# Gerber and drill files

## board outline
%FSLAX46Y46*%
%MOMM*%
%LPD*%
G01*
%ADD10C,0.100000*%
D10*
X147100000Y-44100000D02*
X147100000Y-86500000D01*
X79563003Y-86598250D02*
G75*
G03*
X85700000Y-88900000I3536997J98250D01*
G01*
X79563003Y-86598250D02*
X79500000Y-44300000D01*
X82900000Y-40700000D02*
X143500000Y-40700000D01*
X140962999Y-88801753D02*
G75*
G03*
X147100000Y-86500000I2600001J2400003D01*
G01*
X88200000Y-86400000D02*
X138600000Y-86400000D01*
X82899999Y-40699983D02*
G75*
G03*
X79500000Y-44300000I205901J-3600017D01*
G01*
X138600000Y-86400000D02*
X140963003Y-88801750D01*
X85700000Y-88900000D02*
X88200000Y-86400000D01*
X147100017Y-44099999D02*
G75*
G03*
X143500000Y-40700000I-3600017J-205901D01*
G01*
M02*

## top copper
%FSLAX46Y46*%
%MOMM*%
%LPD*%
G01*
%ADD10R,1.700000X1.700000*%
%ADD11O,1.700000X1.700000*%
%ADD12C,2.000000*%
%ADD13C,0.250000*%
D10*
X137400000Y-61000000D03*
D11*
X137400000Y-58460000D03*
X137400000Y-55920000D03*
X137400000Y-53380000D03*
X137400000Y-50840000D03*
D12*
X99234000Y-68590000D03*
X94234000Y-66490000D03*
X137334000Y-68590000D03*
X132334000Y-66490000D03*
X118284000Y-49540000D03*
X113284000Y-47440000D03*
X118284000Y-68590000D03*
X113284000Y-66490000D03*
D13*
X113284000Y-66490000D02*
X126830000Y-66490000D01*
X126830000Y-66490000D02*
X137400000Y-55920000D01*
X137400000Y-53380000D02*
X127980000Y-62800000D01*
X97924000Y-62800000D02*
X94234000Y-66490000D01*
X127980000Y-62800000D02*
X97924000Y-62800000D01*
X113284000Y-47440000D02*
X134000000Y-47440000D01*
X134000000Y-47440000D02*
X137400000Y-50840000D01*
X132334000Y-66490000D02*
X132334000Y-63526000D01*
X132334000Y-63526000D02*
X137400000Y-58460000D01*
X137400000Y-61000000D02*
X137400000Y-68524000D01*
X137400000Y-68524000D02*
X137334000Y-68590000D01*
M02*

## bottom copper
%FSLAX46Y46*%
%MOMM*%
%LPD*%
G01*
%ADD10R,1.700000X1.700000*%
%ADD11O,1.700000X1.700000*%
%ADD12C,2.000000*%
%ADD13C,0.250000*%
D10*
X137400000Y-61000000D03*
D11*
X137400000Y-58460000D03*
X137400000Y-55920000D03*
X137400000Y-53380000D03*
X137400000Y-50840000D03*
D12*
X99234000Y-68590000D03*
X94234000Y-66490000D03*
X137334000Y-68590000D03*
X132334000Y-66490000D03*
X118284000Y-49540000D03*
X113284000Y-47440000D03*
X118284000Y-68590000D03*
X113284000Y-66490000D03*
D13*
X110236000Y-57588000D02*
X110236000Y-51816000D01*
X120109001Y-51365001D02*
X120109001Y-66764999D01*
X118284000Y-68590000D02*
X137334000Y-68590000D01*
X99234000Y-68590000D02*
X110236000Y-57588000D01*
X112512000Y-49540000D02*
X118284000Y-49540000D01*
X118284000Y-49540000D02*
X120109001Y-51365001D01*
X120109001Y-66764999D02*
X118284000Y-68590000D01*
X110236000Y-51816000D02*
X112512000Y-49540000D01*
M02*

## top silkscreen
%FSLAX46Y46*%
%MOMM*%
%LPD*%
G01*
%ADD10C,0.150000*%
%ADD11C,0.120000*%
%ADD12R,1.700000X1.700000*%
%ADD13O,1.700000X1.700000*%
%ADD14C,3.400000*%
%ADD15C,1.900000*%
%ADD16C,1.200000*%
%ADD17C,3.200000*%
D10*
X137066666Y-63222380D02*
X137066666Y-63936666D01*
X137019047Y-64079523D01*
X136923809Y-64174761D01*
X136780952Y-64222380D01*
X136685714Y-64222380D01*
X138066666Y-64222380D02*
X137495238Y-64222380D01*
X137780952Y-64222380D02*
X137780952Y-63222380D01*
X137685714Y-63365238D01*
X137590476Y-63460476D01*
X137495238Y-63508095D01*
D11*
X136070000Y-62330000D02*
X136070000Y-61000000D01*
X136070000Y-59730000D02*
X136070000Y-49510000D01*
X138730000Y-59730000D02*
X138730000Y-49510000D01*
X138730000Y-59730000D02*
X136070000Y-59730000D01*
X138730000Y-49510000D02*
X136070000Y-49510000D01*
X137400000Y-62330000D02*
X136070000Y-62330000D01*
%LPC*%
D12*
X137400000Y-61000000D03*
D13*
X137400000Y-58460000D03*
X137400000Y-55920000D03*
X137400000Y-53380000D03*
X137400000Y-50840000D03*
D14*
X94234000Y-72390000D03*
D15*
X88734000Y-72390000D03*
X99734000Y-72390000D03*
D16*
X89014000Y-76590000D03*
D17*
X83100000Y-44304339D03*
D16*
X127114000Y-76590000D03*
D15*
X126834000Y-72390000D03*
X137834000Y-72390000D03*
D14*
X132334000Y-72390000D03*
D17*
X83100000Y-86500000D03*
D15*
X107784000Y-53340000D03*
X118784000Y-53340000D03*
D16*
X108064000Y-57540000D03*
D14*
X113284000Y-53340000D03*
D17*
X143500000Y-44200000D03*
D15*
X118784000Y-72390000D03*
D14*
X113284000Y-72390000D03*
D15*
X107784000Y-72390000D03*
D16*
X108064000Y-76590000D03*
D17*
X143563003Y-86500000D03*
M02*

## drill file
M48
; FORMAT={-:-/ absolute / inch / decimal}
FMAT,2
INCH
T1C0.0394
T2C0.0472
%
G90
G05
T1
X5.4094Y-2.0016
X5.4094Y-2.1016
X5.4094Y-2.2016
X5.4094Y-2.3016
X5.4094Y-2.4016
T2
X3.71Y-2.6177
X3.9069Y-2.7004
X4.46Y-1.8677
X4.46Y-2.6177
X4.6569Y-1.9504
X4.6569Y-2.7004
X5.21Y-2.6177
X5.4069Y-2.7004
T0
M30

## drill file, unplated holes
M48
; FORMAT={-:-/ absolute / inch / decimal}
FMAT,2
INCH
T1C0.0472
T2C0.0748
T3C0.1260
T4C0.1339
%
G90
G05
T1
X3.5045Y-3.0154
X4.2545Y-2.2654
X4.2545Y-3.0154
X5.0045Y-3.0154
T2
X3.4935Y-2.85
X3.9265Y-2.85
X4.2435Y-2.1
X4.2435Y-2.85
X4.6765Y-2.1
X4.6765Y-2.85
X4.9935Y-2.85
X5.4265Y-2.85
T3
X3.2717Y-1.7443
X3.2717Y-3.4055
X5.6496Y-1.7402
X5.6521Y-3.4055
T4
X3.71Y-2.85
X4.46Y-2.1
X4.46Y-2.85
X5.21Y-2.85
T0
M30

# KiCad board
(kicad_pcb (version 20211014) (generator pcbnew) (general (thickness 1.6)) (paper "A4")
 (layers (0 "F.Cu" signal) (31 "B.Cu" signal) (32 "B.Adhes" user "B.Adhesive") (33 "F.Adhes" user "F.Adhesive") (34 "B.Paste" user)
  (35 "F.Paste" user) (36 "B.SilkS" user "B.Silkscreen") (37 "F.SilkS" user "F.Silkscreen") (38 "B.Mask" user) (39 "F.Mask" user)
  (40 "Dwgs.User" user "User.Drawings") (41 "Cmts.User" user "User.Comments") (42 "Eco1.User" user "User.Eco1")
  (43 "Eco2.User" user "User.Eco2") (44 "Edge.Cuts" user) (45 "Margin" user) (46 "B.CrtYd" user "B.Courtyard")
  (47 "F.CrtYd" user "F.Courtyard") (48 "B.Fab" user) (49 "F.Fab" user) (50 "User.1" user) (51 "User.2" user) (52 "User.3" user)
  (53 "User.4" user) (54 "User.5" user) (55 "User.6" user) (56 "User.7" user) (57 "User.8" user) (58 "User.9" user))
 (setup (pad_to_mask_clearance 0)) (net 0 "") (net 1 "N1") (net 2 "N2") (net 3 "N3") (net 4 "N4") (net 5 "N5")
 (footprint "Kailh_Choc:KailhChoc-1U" (layer "F.Cu") (at 94.234 72.39)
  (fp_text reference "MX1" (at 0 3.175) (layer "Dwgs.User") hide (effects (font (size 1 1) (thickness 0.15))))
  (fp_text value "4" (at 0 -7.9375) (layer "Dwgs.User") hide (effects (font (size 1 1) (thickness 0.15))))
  (pad "" np_thru_hole circle (at 0 0) (size 3.4 3.4) (drill 3.4) (layers *.Cu *.Mask))
  (pad "" np_thru_hole circle (at -5.5 0 48.1) (size 1.9 1.9) (drill 1.9) (layers *.Cu *.Mask))
  (pad "" np_thru_hole circle (at 5.5 0 48.1) (size 1.9 1.9) (drill 1.9) (layers *.Cu *.Mask))
  (pad "" np_thru_hole circle (at -5.22 4.2) (size 1.2 1.2) (drill 1.2) (layers *.Cu *.Mask))
  (pad "1" thru_hole circle (at 5 -3.8) (size 2 2) (drill 1.2) (layers *.Cu "B.Mask") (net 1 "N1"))
  (pad "2" thru_hole circle (at 0 -5.9) (size 2 2) (drill 1.2) (layers *.Cu "B.Mask") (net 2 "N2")))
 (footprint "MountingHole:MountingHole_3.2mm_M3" (layer "F.Cu") (at 83.1 44.304339)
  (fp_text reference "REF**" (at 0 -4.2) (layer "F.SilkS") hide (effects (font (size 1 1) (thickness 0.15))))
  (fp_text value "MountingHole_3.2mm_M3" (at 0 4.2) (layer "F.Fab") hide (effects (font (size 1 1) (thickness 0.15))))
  (pad "" np_thru_hole circle locked (at 0 0) (size 3.2 3.2) (drill 3.2) (layers F&B.Cu *.Mask)))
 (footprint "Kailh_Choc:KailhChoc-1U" (layer "F.Cu") (at 132.334 72.39)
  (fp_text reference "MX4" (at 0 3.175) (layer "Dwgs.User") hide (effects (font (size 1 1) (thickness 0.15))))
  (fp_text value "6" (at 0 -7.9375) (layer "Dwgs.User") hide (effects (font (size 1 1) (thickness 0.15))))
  (pad "" np_thru_hole circle (at -5.22 4.2) (size 1.2 1.2) (drill 1.2) (layers *.Cu *.Mask))
  (pad "" np_thru_hole circle (at -5.5 0 48.1) (size 1.9 1.9) (drill 1.9) (layers *.Cu *.Mask))
  (pad "" np_thru_hole circle (at 5.5 0 48.1) (size 1.9 1.9) (drill 1.9) (layers *.Cu *.Mask))
  (pad "" np_thru_hole circle (at 0 0) (size 3.4 3.4) (drill 3.4) (layers *.Cu *.Mask))
  (pad "1" thru_hole circle (at 5 -3.8) (size 2 2) (drill 1.2) (layers *.Cu "B.Mask") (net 1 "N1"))
  (pad "2" thru_hole circle (at 0 -5.9) (size 2 2) (drill 1.2) (layers *.Cu "B.Mask") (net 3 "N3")))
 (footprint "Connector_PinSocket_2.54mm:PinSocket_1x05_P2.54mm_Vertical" (layer "F.Cu") (at 137.4 61 180)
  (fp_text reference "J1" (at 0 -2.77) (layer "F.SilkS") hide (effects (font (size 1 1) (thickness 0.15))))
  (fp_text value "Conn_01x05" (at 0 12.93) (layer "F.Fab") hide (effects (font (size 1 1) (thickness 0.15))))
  (fp_line (start -1.33 1.27) (end 1.33 1.27) (layer "F.SilkS") (width 0.12))
  (fp_line (start -1.33 11.49) (end 1.33 11.49) (layer "F.SilkS") (width 0.12))
  (fp_line (start 1.33 1.27) (end 1.33 11.49) (layer "F.SilkS") (width 0.12))
  (fp_line (start 0 -1.33) (end 1.33 -1.33) (layer "F.SilkS") (width 0.12))
  (fp_line (start -1.33 1.27) (end -1.33 11.49) (layer "F.SilkS") (width 0.12))
  (fp_line (start 1.33 -1.33) (end 1.33 0) (layer "F.SilkS") (width 0.12))
  (pad "1" thru_hole rect (at 0 0 180) (size 1.7 1.7) (drill 1) (layers *.Cu *.Mask) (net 1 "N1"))
  (pad "2" thru_hole oval (at 0 2.54 180) (size 1.7 1.7) (drill 1) (layers *.Cu *.Mask) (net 3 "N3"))
  (pad "3" thru_hole oval (at 0 5.08 180) (size 1.7 1.7) (drill 1) (layers *.Cu *.Mask) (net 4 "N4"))
  (pad "4" thru_hole oval (at 0 7.62 180) (size 1.7 1.7) (drill 1) (layers *.Cu *.Mask) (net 2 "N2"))
  (pad "5" thru_hole oval (at 0 10.16 180) (size 1.7 1.7) (drill 1) (layers *.Cu *.Mask) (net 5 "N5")))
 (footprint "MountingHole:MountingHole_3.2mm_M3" (layer "F.Cu") (at 83.1 86.5)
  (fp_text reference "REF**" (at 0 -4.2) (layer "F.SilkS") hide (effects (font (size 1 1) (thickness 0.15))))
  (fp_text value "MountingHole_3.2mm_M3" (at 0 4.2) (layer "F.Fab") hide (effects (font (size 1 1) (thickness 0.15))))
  (pad "" np_thru_hole circle locked (at 0 0) (size 3.2 3.2) (drill 3.2) (layers *.Cu *.Mask)))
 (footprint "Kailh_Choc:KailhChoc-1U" (layer "F.Cu") (at 113.284 53.34)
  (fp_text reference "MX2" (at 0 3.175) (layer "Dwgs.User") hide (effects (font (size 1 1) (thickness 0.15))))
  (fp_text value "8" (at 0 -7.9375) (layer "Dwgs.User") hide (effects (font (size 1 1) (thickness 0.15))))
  (pad "" np_thru_hole circle (at -5.5 0 48.1) (size 1.9 1.9) (drill 1.9) (layers *.Cu *.Mask))
  (pad "" np_thru_hole circle (at 5.5 0 48.1) (size 1.9 1.9) (drill 1.9) (layers *.Cu *.Mask))
  (pad "" np_thru_hole circle (at -5.22 4.2) (size 1.2 1.2) (drill 1.2) (layers *.Cu *.Mask))
  (pad "" np_thru_hole circle (at 0 0) (size 3.4 3.4) (drill 3.4) (layers *.Cu *.Mask))
  (pad "1" thru_hole circle (at 5 -3.8) (size 2 2) (drill 1.2) (layers *.Cu "B.Mask") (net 1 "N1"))
  (pad "2" thru_hole circle (at 0 -5.9) (size 2 2) (drill 1.2) (layers *.Cu "B.Mask") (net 5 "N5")))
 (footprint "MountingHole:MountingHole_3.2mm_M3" (layer "F.Cu") (at 143.5 44.2)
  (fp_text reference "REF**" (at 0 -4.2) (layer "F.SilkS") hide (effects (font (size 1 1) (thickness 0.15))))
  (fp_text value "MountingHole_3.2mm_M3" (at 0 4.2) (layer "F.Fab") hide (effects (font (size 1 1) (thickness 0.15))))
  (pad "" np_thru_hole circle locked (at 0 0) (size 3.2 3.2) (drill 3.2) (layers F&B.Cu *.Mask)))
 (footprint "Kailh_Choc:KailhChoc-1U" (layer "F.Cu") (at 113.284 72.39)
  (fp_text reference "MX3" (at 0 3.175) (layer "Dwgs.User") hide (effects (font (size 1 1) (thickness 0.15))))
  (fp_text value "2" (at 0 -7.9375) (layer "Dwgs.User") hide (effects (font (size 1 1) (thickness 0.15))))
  (pad "" np_thru_hole circle (at 5.5 0 48.1) (size 1.9 1.9) (drill 1.9) (layers *.Cu *.Mask))
  (pad "" np_thru_hole circle (at 0 0) (size 3.4 3.4) (drill 3.4) (layers *.Cu *.Mask))
  (pad "" np_thru_hole circle (at -5.5 0 48.1) (size 1.9 1.9) (drill 1.9) (layers *.Cu *.Mask))
  (pad "" np_thru_hole circle (at -5.22 4.2) (size 1.2 1.2) (drill 1.2) (layers *.Cu *.Mask))
  (pad "1" thru_hole circle (at 5 -3.8) (size 2 2) (drill 1.2) (layers *.Cu "B.Mask") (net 1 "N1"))
  (pad "2" thru_hole circle (at 0 -5.9) (size 2 2) (drill 1.2) (layers *.Cu "B.Mask") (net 4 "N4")))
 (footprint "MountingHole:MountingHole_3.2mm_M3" (layer "B.Cu") (at 143.563003 86.5 180)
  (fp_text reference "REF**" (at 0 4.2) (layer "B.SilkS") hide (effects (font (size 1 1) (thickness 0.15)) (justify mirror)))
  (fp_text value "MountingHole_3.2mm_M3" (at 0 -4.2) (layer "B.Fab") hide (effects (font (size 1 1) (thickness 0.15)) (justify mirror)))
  (pad "" np_thru_hole circle locked (at 0 0 180) (size 3.2 3.2) (drill 3.2) (layers F&B.Cu *.Mask)))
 (gr_line (start 147.1 44.1) (end 147.1 86.5) (layer "Edge.Cuts") (width 0.1))
 (gr_arc (start 85.7 88.9) (mid 81.85742 89.813004) (end 79.563003 86.59825) (layer "Edge.Cuts") (width 0.1))
 (gr_line (start 79.563003 86.59825) (end 79.5 44.3) (layer "Edge.Cuts") (width 0.1))
 (gr_line (start 82.9 40.7) (end 143.5 40.7) (layer "Edge.Cuts") (width 0.1))
 (gr_arc (start 147.1 86.5) (mid 144.805583 89.714754) (end 140.963003 88.80175) (layer "Edge.Cuts") (width 0.1))
 (gr_line (start 88.2 86.4) (end 138.6 86.4) (layer "Edge.Cuts") (width 0.1))
 (gr_arc (start 79.5 44.3) (mid 80.484358 41.824116) (end 82.9 40.7) (layer "Edge.Cuts") (width 0.1))
 (gr_line (start 138.6 86.4) (end 140.963003 88.80175) (layer "Edge.Cuts") (width 0.1))
 (gr_line (start 85.7 88.9) (end 88.2 86.4) (layer "Edge.Cuts") (width 0.1))
 (gr_arc (start 143.5 40.7) (mid 145.975884 41.684358) (end 147.1 44.1) (layer "Edge.Cuts") (width 0.1))
 (segment (start 137.4 68.524) (end 137.334 68.59) (width 0.25) (layer "F.Cu") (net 1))
 (segment (start 137.4 61) (end 137.4 68.524) (width 0.25) (layer "F.Cu") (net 1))
 (segment (start 110.236 57.588) (end 110.236 51.816) (width 0.25) (layer "B.Cu") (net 1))
 (segment (start 120.109001 51.365001) (end 120.109001 66.764999) (width 0.25) (layer "B.Cu") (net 1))
 (segment (start 118.284 68.59) (end 137.334 68.59) (width 0.25) (layer "B.Cu") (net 1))
 (segment (start 99.234 68.59) (end 110.236 57.588) (width 0.25) (layer "B.Cu") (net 1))
 (segment (start 112.512 49.54) (end 118.284 49.54) (width 0.25) (layer "B.Cu") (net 1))
 (segment (start 118.284 49.54) (end 120.109001 51.365001) (width 0.25) (layer "B.Cu") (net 1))
 (segment (start 120.109001 66.764999) (end 118.284 68.59) (width 0.25) (layer "B.Cu") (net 1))
 (segment (start 110.236 51.816) (end 112.512 49.54) (width 0.25) (layer "B.Cu") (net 1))
 (segment (start 132.334 63.526) (end 137.4 58.46) (width 0.25) (layer "F.Cu") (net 3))
 (segment (start 132.334 66.49) (end 132.334 63.526) (width 0.25) (layer "F.Cu") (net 3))
 (segment (start 113.284 66.49) (end 126.83 66.49) (width 0.25) (layer "F.Cu") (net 4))
 (segment (start 126.83 66.49) (end 137.4 55.92) (width 0.25) (layer "F.Cu") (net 4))
 (segment (start 127.98 62.8) (end 97.924 62.8) (width 0.25) (layer "F.Cu") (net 2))
 (segment (start 137.4 53.38) (end 127.98 62.8) (width 0.25) (layer "F.Cu") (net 2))
 (segment (start 97.924 62.8) (end 94.234 66.49) (width 0.25) (layer "F.Cu") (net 2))
 (segment (start 113.284 47.44) (end 134 47.44) (width 0.25) (layer "F.Cu") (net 5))
 (segment (start 134 47.44) (end 137.4 50.84) (width 0.25) (layer "F.Cu") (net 5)))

